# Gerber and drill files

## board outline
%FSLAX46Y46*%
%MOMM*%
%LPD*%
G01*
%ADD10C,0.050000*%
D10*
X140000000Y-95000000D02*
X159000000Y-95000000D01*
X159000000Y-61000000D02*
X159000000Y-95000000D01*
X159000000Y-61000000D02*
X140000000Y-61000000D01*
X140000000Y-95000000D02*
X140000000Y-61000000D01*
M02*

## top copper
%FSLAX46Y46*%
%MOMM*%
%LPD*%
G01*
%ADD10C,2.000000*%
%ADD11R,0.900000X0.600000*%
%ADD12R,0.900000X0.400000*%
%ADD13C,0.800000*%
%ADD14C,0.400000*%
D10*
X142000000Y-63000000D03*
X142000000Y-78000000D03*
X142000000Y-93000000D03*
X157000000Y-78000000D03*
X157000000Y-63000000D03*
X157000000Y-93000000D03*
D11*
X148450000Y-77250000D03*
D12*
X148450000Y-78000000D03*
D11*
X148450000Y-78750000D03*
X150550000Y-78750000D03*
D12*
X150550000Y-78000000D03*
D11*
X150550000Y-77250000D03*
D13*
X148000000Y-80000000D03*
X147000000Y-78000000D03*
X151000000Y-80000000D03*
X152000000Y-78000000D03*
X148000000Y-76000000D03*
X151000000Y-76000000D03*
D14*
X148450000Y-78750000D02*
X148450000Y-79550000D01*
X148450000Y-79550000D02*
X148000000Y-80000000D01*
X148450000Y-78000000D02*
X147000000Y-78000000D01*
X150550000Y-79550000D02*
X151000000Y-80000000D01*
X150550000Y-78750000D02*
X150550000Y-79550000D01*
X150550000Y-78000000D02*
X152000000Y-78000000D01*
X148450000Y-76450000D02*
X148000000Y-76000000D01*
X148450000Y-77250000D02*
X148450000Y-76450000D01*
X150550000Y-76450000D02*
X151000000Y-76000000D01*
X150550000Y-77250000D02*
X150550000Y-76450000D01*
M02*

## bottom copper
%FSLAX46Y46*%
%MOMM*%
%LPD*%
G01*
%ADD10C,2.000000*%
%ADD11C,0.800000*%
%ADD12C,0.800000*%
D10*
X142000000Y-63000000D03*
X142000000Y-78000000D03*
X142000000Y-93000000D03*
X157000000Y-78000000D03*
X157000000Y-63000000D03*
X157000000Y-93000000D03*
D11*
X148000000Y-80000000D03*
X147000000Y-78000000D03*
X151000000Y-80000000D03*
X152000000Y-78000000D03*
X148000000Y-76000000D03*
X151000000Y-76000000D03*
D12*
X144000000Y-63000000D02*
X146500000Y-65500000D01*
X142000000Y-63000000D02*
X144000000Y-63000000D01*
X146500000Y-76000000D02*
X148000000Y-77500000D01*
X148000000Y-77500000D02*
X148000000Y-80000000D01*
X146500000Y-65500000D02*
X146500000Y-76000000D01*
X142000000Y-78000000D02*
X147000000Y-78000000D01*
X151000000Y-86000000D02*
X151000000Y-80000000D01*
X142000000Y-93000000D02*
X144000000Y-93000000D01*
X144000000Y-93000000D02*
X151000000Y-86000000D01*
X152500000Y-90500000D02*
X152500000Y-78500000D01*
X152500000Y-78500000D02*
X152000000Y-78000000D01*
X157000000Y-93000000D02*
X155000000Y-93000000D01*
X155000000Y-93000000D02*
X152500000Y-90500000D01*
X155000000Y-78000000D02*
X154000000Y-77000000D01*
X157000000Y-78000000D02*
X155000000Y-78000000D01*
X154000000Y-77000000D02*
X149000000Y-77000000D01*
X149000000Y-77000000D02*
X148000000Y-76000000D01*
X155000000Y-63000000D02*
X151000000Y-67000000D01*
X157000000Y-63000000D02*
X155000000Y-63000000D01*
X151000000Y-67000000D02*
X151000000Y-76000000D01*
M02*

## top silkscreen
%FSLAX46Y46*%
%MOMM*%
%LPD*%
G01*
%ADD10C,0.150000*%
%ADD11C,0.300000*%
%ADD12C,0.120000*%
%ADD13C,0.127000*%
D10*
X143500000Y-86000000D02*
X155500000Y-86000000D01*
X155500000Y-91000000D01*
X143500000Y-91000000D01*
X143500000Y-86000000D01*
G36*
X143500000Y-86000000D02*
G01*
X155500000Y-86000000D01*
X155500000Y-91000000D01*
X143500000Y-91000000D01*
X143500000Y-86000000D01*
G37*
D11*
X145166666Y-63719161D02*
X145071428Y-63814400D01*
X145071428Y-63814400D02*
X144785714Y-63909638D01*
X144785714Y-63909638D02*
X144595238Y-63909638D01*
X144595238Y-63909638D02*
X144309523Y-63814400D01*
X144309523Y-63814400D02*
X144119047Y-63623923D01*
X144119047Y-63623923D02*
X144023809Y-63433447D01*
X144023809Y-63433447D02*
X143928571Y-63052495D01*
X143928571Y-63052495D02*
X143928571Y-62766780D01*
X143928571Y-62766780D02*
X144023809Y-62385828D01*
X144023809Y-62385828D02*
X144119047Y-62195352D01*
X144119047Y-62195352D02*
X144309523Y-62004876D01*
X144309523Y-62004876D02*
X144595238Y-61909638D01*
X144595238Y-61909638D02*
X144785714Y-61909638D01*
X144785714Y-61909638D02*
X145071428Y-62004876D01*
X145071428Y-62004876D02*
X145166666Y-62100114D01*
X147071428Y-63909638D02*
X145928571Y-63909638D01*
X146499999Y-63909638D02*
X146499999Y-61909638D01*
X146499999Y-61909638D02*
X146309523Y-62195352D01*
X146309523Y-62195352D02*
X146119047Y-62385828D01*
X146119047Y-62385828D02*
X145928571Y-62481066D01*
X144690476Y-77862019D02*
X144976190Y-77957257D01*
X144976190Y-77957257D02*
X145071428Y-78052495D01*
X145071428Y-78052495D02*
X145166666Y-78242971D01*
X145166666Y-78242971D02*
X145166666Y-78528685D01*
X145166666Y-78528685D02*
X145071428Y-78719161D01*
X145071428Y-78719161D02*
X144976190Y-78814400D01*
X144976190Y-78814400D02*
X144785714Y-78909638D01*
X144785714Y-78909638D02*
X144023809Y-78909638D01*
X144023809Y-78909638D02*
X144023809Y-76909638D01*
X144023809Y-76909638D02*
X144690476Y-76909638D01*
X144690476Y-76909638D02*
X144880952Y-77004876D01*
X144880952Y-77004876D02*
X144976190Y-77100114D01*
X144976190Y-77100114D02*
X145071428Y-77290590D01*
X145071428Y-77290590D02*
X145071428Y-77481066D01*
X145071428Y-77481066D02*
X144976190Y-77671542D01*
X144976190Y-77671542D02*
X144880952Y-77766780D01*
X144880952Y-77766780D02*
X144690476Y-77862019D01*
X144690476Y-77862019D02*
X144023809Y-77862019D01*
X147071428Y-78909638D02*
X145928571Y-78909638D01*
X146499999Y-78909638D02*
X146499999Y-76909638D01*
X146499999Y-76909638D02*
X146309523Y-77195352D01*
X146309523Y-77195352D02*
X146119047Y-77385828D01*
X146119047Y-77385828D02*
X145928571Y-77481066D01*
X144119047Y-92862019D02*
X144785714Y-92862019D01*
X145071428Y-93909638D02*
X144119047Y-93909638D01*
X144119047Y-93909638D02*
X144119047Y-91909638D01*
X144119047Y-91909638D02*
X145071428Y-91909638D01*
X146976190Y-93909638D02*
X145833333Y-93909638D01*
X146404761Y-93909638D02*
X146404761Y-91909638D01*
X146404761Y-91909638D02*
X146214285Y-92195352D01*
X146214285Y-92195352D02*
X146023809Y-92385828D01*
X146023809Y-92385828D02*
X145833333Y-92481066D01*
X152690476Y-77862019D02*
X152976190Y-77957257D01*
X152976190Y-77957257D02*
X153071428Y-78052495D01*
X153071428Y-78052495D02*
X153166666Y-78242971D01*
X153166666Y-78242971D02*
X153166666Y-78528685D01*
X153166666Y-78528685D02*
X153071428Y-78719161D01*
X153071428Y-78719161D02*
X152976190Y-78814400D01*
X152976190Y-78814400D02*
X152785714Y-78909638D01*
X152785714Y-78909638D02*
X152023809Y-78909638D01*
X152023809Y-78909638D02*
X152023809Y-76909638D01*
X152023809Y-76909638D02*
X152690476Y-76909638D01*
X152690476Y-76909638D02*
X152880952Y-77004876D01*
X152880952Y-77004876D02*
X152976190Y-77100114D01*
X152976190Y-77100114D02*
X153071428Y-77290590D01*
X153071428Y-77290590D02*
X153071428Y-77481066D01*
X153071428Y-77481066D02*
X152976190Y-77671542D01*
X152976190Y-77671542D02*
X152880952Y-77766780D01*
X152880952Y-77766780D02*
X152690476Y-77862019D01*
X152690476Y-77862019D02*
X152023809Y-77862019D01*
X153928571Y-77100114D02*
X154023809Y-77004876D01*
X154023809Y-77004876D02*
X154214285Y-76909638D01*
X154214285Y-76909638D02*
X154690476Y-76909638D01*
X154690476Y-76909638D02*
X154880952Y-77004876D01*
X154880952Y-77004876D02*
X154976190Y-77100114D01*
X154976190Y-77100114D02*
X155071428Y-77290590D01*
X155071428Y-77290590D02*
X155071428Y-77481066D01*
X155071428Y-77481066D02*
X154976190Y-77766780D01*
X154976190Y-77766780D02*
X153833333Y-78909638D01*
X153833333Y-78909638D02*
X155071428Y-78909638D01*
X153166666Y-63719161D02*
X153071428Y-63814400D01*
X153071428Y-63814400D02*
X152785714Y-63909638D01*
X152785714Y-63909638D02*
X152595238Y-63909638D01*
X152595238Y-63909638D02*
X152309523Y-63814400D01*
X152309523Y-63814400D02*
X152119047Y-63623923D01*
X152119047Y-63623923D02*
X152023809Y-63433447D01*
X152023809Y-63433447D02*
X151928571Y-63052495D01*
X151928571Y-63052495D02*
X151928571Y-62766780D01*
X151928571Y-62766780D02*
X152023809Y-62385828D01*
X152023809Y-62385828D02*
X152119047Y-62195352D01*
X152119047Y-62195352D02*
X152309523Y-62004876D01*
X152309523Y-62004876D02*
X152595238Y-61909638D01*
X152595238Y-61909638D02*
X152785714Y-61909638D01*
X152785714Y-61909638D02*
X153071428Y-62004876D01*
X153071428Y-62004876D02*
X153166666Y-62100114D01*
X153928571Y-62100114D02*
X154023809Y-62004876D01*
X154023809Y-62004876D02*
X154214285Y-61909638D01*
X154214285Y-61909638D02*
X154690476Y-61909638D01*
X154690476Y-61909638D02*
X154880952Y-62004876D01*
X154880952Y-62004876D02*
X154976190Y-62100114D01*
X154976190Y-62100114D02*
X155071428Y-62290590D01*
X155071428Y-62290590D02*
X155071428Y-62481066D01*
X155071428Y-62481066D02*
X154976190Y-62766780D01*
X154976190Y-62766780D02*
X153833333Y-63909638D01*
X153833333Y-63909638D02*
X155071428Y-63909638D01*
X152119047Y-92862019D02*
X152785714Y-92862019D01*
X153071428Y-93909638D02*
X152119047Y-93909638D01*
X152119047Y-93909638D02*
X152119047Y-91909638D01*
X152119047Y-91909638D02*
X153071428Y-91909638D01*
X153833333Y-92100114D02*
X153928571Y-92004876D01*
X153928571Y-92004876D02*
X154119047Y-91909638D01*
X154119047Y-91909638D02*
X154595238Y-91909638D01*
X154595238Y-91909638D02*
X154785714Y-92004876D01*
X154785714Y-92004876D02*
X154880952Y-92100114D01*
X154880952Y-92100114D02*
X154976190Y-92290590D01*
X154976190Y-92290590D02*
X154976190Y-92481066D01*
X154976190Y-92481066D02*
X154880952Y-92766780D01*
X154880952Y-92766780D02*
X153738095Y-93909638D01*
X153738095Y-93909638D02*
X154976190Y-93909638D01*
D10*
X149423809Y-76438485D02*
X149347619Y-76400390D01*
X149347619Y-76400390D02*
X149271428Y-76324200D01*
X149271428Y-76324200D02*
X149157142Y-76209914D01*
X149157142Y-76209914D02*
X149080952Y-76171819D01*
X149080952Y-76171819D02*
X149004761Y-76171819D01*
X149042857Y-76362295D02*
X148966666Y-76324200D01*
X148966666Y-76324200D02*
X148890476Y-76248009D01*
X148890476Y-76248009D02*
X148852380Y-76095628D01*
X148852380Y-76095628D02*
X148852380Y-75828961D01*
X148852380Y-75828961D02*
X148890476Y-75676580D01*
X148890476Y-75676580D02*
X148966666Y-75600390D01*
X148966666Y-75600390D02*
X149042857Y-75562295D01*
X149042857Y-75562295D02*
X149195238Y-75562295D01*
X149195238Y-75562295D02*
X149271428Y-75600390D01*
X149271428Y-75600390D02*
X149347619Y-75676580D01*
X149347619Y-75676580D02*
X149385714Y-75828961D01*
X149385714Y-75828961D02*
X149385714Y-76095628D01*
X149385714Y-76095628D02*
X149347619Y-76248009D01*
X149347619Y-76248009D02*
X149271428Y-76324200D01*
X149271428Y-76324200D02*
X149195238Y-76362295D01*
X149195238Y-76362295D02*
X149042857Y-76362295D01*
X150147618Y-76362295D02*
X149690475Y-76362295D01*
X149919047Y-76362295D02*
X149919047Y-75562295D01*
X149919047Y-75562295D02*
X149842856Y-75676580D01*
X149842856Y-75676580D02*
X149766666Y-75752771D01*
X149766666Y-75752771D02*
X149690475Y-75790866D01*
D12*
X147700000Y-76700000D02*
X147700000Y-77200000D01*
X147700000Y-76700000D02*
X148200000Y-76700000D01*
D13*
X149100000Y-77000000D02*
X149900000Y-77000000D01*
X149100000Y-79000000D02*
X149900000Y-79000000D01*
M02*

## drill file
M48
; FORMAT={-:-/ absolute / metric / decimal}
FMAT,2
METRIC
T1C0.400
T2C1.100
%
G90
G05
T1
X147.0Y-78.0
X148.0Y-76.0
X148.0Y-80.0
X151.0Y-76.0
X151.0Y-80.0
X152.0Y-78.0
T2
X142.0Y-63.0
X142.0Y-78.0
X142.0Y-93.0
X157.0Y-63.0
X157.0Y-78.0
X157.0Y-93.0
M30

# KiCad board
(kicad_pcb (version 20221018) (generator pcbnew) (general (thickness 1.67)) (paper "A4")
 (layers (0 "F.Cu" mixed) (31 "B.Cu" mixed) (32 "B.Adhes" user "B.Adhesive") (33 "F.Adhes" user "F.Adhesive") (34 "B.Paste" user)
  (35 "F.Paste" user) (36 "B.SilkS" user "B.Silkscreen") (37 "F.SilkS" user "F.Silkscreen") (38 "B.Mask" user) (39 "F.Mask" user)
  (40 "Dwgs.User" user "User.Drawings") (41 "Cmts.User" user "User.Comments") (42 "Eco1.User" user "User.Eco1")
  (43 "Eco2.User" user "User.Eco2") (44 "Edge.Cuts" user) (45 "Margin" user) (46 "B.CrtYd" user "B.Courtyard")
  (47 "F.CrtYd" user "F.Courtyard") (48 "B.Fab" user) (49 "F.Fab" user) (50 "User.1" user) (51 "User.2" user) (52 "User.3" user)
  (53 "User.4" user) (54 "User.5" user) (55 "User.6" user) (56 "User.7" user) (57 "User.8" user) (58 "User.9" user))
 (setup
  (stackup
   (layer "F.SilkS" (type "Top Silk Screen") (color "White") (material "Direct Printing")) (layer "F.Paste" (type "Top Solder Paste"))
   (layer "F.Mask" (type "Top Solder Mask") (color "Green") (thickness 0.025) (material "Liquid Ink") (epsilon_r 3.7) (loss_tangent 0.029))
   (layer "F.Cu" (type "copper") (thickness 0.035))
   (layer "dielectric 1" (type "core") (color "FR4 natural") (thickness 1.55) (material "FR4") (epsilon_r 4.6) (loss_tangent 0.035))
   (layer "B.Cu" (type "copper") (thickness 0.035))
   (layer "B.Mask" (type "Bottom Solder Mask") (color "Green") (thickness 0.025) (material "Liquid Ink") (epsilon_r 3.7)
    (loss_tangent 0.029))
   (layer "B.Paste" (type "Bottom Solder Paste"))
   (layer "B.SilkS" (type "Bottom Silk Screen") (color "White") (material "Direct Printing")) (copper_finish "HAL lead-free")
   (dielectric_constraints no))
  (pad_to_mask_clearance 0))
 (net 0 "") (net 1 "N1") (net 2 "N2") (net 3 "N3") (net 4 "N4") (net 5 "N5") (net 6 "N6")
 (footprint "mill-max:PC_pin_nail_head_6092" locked (layer "F.Cu") (at 142 63)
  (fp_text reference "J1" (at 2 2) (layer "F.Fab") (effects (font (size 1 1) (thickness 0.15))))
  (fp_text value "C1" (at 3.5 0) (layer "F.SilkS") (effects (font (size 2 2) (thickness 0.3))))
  (pad "1" thru_hole circle locked (at 0 0) (size 2 2) (drill 1.1) (layers "*.Cu" "*.Mask") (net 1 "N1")))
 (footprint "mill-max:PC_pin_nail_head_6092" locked (layer "F.Cu") (at 142 78)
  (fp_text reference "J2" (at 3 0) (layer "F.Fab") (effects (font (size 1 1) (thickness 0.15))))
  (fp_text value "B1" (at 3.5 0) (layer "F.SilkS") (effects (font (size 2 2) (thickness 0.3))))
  (pad "1" thru_hole circle locked (at 0 0) (size 2 2) (drill 1.1) (layers "*.Cu" "*.Mask") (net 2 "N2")))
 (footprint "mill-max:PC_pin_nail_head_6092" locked (layer "F.Cu") (at 142 93)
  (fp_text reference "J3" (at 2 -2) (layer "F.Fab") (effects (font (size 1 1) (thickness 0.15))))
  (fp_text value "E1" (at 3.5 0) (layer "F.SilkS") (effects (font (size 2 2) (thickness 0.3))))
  (pad "1" thru_hole circle locked (at 0 0) (size 2 2) (drill 1.1) (layers "*.Cu" "*.Mask") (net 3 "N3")))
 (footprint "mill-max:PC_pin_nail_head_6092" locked (layer "F.Cu") (at 157 78)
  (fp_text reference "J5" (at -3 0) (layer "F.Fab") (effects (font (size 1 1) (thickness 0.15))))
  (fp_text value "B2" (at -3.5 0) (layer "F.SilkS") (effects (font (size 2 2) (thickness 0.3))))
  (pad "1" thru_hole circle locked (at 0 0) (size 2 2) (drill 1.1) (layers "*.Cu" "*.Mask") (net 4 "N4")))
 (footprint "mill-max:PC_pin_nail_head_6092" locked (layer "F.Cu") (at 157 63)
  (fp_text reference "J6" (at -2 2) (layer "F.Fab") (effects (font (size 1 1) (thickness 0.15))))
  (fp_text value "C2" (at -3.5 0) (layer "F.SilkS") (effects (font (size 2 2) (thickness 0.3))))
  (pad "1" thru_hole circle locked (at 0 0) (size 2 2) (drill 1.1) (layers "*.Cu" "*.Mask") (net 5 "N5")))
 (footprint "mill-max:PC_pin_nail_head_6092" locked (layer "F.Cu") (at 157 93)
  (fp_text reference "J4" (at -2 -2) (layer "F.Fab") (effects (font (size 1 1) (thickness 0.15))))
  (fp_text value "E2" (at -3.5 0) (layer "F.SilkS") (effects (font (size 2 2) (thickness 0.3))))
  (pad "1" thru_hole circle locked (at 0 0) (size 2 2) (drill 1.1) (layers "*.Cu" "*.Mask") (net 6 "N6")))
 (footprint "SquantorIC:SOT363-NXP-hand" (layer "F.Cu") (at 149.5 78)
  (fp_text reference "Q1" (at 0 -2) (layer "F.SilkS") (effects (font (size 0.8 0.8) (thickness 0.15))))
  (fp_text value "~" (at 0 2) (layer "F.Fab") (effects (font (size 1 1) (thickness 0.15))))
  (fp_line (start -1.8 -1.3) (end -1.8 -0.8) (stroke (width 0.12) (type solid)) (layer "F.SilkS"))
  (fp_line (start -1.8 -1.3) (end -1.3 -1.3) (stroke (width 0.12) (type solid)) (layer "F.SilkS"))
  (fp_line (start -0.4 -1) (end 0.4 -1) (stroke (width 0.127) (type solid)) (layer "F.SilkS"))
  (fp_line (start -0.4 1) (end 0.4 1) (stroke (width 0.127) (type solid)) (layer "F.SilkS"))
  (pad "1" smd rect (at -1.05 -0.75 270) (size 0.6 0.9) (layers "F.Cu" "F.Paste" "F.Mask") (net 4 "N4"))
  (pad "2" smd rect (at -1.05 0 270) (size 0.4 0.9) (layers "F.Cu" "F.Paste" "F.Mask") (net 2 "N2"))
  (pad "3" smd rect (at -1.05 0.75 270) (size 0.6 0.9) (layers "F.Cu" "F.Paste" "F.Mask") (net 1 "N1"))
  (pad "4" smd rect (at 1.05 0.75 270) (size 0.6 0.9) (layers "F.Cu" "F.Paste" "F.Mask") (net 3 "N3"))
  (pad "5" smd rect (at 1.05 0 270) (size 0.4 0.9) (layers "F.Cu" "F.Paste" "F.Mask") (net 6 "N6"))
  (pad "6" smd rect (at 1.05 -0.75 270) (size 0.6 0.9) (layers "F.Cu" "F.Paste" "F.Mask") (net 5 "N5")))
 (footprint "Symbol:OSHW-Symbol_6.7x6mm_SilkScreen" (layer "B.Cu") (at 149 90 180)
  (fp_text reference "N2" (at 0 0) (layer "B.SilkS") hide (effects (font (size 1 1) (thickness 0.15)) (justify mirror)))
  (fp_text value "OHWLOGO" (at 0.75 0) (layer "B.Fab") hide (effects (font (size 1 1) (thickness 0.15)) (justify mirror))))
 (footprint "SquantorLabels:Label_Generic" (layer "B.Cu") (at 148.5 93.5)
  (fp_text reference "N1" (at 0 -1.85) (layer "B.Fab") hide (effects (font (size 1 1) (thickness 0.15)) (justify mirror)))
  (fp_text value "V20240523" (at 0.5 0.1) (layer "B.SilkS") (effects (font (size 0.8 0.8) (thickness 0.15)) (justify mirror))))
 (gr_rect (start 143.5 86) (end 155.5 91) (stroke (width 0.15) (type solid)) (fill solid) (layer "F.SilkS"))
 (gr_line (start 140 95) (end 159 95) (stroke (width 0.05) (type solid)) (layer "Edge.Cuts"))
 (gr_line (start 159 61) (end 159 95) (stroke (width 0.05) (type solid)) (layer "Edge.Cuts"))
 (gr_line (start 159 61) (end 140 61) (stroke (width 0.05) (type solid)) (layer "Edge.Cuts"))
 (gr_line (start 140 95) (end 140 61) (stroke (width 0.05) (type solid)) (layer "Edge.Cuts"))
 (segment (start 148.45 78.75) (end 148.45 79.55) (width 0.4) (layer "F.Cu") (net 1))
 (segment (start 148.45 79.55) (end 148 80) (width 0.4) (layer "F.Cu") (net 1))
 (via (at 148 80) (size 0.8) (drill 0.4) (layers "F.Cu" "B.Cu") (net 1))
 (segment (start 144 63) (end 146.5 65.5) (width 0.8) (layer "B.Cu") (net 1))
 (segment (start 142 63) (end 144 63) (width 0.8) (layer "B.Cu") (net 1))
 (segment (start 146.5 76) (end 148 77.5) (width 0.8) (layer "B.Cu") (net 1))
 (segment (start 148 77.5) (end 148 80) (width 0.8) (layer "B.Cu") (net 1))
 (segment (start 146.5 65.5) (end 146.5 76) (width 0.8) (layer "B.Cu") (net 1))
 (segment (start 148.45 78) (end 147 78) (width 0.4) (layer "F.Cu") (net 2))
 (via (at 147 78) (size 0.8) (drill 0.4) (layers "F.Cu" "B.Cu") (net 2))
 (segment (start 142 78) (end 147 78) (width 0.8) (layer "B.Cu") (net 2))
 (segment (start 150.55 79.55) (end 151 80) (width 0.4) (layer "F.Cu") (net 3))
 (segment (start 150.55 78.75) (end 150.55 79.55) (width 0.4) (layer "F.Cu") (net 3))
 (via (at 151 80) (size 0.8) (drill 0.4) (layers "F.Cu" "B.Cu") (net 3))
 (segment (start 151 86) (end 151 80) (width 0.8) (layer "B.Cu") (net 3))
 (segment (start 142 93) (end 144 93) (width 0.8) (layer "B.Cu") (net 3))
 (segment (start 144 93) (end 151 86) (width 0.8) (layer "B.Cu") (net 3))
 (segment (start 150.55 78) (end 152 78) (width 0.4) (layer "F.Cu") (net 6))
 (via (at 152 78) (size 0.8) (drill 0.4) (layers "F.Cu" "B.Cu") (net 6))
 (segment (start 152.5 90.5) (end 152.5 78.5) (width 0.8) (layer "B.Cu") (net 6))
 (segment (start 152.5 78.5) (end 152 78) (width 0.8) (layer "B.Cu") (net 6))
 (segment (start 157 93) (end 155 93) (width 0.8) (layer "B.Cu") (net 6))
 (segment (start 155 93) (end 152.5 90.5) (width 0.8) (layer "B.Cu") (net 6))
 (segment (start 148.45 76.45) (end 148 76) (width 0.4) (layer "F.Cu") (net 4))
 (segment (start 148.45 77.25) (end 148.45 76.45) (width 0.4) (layer "F.Cu") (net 4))
 (via (at 148 76) (size 0.8) (drill 0.4) (layers "F.Cu" "B.Cu") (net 4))
 (segment (start 155 78) (end 154 77) (width 0.8) (layer "B.Cu") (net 4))
 (segment (start 157 78) (end 155 78) (width 0.8) (layer "B.Cu") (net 4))
 (segment (start 154 77) (end 149 77) (width 0.8) (layer "B.Cu") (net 4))
 (segment (start 149 77) (end 148 76) (width 0.8) (layer "B.Cu") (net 4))
 (segment (start 150.55 76.45) (end 151 76) (width 0.4) (layer "F.Cu") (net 5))
 (segment (start 150.55 77.25) (end 150.55 76.45) (width 0.4) (layer "F.Cu") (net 5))
 (via (at 151 76) (size 0.8) (drill 0.4) (layers "F.Cu" "B.Cu") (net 5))
 (segment (start 155 63) (end 151 67) (width 0.8) (layer "B.Cu") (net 5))
 (segment (start 157 63) (end 155 63) (width 0.8) (layer "B.Cu") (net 5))
 (segment (start 151 67) (end 151 76) (width 0.8) (layer "B.Cu") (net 5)))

